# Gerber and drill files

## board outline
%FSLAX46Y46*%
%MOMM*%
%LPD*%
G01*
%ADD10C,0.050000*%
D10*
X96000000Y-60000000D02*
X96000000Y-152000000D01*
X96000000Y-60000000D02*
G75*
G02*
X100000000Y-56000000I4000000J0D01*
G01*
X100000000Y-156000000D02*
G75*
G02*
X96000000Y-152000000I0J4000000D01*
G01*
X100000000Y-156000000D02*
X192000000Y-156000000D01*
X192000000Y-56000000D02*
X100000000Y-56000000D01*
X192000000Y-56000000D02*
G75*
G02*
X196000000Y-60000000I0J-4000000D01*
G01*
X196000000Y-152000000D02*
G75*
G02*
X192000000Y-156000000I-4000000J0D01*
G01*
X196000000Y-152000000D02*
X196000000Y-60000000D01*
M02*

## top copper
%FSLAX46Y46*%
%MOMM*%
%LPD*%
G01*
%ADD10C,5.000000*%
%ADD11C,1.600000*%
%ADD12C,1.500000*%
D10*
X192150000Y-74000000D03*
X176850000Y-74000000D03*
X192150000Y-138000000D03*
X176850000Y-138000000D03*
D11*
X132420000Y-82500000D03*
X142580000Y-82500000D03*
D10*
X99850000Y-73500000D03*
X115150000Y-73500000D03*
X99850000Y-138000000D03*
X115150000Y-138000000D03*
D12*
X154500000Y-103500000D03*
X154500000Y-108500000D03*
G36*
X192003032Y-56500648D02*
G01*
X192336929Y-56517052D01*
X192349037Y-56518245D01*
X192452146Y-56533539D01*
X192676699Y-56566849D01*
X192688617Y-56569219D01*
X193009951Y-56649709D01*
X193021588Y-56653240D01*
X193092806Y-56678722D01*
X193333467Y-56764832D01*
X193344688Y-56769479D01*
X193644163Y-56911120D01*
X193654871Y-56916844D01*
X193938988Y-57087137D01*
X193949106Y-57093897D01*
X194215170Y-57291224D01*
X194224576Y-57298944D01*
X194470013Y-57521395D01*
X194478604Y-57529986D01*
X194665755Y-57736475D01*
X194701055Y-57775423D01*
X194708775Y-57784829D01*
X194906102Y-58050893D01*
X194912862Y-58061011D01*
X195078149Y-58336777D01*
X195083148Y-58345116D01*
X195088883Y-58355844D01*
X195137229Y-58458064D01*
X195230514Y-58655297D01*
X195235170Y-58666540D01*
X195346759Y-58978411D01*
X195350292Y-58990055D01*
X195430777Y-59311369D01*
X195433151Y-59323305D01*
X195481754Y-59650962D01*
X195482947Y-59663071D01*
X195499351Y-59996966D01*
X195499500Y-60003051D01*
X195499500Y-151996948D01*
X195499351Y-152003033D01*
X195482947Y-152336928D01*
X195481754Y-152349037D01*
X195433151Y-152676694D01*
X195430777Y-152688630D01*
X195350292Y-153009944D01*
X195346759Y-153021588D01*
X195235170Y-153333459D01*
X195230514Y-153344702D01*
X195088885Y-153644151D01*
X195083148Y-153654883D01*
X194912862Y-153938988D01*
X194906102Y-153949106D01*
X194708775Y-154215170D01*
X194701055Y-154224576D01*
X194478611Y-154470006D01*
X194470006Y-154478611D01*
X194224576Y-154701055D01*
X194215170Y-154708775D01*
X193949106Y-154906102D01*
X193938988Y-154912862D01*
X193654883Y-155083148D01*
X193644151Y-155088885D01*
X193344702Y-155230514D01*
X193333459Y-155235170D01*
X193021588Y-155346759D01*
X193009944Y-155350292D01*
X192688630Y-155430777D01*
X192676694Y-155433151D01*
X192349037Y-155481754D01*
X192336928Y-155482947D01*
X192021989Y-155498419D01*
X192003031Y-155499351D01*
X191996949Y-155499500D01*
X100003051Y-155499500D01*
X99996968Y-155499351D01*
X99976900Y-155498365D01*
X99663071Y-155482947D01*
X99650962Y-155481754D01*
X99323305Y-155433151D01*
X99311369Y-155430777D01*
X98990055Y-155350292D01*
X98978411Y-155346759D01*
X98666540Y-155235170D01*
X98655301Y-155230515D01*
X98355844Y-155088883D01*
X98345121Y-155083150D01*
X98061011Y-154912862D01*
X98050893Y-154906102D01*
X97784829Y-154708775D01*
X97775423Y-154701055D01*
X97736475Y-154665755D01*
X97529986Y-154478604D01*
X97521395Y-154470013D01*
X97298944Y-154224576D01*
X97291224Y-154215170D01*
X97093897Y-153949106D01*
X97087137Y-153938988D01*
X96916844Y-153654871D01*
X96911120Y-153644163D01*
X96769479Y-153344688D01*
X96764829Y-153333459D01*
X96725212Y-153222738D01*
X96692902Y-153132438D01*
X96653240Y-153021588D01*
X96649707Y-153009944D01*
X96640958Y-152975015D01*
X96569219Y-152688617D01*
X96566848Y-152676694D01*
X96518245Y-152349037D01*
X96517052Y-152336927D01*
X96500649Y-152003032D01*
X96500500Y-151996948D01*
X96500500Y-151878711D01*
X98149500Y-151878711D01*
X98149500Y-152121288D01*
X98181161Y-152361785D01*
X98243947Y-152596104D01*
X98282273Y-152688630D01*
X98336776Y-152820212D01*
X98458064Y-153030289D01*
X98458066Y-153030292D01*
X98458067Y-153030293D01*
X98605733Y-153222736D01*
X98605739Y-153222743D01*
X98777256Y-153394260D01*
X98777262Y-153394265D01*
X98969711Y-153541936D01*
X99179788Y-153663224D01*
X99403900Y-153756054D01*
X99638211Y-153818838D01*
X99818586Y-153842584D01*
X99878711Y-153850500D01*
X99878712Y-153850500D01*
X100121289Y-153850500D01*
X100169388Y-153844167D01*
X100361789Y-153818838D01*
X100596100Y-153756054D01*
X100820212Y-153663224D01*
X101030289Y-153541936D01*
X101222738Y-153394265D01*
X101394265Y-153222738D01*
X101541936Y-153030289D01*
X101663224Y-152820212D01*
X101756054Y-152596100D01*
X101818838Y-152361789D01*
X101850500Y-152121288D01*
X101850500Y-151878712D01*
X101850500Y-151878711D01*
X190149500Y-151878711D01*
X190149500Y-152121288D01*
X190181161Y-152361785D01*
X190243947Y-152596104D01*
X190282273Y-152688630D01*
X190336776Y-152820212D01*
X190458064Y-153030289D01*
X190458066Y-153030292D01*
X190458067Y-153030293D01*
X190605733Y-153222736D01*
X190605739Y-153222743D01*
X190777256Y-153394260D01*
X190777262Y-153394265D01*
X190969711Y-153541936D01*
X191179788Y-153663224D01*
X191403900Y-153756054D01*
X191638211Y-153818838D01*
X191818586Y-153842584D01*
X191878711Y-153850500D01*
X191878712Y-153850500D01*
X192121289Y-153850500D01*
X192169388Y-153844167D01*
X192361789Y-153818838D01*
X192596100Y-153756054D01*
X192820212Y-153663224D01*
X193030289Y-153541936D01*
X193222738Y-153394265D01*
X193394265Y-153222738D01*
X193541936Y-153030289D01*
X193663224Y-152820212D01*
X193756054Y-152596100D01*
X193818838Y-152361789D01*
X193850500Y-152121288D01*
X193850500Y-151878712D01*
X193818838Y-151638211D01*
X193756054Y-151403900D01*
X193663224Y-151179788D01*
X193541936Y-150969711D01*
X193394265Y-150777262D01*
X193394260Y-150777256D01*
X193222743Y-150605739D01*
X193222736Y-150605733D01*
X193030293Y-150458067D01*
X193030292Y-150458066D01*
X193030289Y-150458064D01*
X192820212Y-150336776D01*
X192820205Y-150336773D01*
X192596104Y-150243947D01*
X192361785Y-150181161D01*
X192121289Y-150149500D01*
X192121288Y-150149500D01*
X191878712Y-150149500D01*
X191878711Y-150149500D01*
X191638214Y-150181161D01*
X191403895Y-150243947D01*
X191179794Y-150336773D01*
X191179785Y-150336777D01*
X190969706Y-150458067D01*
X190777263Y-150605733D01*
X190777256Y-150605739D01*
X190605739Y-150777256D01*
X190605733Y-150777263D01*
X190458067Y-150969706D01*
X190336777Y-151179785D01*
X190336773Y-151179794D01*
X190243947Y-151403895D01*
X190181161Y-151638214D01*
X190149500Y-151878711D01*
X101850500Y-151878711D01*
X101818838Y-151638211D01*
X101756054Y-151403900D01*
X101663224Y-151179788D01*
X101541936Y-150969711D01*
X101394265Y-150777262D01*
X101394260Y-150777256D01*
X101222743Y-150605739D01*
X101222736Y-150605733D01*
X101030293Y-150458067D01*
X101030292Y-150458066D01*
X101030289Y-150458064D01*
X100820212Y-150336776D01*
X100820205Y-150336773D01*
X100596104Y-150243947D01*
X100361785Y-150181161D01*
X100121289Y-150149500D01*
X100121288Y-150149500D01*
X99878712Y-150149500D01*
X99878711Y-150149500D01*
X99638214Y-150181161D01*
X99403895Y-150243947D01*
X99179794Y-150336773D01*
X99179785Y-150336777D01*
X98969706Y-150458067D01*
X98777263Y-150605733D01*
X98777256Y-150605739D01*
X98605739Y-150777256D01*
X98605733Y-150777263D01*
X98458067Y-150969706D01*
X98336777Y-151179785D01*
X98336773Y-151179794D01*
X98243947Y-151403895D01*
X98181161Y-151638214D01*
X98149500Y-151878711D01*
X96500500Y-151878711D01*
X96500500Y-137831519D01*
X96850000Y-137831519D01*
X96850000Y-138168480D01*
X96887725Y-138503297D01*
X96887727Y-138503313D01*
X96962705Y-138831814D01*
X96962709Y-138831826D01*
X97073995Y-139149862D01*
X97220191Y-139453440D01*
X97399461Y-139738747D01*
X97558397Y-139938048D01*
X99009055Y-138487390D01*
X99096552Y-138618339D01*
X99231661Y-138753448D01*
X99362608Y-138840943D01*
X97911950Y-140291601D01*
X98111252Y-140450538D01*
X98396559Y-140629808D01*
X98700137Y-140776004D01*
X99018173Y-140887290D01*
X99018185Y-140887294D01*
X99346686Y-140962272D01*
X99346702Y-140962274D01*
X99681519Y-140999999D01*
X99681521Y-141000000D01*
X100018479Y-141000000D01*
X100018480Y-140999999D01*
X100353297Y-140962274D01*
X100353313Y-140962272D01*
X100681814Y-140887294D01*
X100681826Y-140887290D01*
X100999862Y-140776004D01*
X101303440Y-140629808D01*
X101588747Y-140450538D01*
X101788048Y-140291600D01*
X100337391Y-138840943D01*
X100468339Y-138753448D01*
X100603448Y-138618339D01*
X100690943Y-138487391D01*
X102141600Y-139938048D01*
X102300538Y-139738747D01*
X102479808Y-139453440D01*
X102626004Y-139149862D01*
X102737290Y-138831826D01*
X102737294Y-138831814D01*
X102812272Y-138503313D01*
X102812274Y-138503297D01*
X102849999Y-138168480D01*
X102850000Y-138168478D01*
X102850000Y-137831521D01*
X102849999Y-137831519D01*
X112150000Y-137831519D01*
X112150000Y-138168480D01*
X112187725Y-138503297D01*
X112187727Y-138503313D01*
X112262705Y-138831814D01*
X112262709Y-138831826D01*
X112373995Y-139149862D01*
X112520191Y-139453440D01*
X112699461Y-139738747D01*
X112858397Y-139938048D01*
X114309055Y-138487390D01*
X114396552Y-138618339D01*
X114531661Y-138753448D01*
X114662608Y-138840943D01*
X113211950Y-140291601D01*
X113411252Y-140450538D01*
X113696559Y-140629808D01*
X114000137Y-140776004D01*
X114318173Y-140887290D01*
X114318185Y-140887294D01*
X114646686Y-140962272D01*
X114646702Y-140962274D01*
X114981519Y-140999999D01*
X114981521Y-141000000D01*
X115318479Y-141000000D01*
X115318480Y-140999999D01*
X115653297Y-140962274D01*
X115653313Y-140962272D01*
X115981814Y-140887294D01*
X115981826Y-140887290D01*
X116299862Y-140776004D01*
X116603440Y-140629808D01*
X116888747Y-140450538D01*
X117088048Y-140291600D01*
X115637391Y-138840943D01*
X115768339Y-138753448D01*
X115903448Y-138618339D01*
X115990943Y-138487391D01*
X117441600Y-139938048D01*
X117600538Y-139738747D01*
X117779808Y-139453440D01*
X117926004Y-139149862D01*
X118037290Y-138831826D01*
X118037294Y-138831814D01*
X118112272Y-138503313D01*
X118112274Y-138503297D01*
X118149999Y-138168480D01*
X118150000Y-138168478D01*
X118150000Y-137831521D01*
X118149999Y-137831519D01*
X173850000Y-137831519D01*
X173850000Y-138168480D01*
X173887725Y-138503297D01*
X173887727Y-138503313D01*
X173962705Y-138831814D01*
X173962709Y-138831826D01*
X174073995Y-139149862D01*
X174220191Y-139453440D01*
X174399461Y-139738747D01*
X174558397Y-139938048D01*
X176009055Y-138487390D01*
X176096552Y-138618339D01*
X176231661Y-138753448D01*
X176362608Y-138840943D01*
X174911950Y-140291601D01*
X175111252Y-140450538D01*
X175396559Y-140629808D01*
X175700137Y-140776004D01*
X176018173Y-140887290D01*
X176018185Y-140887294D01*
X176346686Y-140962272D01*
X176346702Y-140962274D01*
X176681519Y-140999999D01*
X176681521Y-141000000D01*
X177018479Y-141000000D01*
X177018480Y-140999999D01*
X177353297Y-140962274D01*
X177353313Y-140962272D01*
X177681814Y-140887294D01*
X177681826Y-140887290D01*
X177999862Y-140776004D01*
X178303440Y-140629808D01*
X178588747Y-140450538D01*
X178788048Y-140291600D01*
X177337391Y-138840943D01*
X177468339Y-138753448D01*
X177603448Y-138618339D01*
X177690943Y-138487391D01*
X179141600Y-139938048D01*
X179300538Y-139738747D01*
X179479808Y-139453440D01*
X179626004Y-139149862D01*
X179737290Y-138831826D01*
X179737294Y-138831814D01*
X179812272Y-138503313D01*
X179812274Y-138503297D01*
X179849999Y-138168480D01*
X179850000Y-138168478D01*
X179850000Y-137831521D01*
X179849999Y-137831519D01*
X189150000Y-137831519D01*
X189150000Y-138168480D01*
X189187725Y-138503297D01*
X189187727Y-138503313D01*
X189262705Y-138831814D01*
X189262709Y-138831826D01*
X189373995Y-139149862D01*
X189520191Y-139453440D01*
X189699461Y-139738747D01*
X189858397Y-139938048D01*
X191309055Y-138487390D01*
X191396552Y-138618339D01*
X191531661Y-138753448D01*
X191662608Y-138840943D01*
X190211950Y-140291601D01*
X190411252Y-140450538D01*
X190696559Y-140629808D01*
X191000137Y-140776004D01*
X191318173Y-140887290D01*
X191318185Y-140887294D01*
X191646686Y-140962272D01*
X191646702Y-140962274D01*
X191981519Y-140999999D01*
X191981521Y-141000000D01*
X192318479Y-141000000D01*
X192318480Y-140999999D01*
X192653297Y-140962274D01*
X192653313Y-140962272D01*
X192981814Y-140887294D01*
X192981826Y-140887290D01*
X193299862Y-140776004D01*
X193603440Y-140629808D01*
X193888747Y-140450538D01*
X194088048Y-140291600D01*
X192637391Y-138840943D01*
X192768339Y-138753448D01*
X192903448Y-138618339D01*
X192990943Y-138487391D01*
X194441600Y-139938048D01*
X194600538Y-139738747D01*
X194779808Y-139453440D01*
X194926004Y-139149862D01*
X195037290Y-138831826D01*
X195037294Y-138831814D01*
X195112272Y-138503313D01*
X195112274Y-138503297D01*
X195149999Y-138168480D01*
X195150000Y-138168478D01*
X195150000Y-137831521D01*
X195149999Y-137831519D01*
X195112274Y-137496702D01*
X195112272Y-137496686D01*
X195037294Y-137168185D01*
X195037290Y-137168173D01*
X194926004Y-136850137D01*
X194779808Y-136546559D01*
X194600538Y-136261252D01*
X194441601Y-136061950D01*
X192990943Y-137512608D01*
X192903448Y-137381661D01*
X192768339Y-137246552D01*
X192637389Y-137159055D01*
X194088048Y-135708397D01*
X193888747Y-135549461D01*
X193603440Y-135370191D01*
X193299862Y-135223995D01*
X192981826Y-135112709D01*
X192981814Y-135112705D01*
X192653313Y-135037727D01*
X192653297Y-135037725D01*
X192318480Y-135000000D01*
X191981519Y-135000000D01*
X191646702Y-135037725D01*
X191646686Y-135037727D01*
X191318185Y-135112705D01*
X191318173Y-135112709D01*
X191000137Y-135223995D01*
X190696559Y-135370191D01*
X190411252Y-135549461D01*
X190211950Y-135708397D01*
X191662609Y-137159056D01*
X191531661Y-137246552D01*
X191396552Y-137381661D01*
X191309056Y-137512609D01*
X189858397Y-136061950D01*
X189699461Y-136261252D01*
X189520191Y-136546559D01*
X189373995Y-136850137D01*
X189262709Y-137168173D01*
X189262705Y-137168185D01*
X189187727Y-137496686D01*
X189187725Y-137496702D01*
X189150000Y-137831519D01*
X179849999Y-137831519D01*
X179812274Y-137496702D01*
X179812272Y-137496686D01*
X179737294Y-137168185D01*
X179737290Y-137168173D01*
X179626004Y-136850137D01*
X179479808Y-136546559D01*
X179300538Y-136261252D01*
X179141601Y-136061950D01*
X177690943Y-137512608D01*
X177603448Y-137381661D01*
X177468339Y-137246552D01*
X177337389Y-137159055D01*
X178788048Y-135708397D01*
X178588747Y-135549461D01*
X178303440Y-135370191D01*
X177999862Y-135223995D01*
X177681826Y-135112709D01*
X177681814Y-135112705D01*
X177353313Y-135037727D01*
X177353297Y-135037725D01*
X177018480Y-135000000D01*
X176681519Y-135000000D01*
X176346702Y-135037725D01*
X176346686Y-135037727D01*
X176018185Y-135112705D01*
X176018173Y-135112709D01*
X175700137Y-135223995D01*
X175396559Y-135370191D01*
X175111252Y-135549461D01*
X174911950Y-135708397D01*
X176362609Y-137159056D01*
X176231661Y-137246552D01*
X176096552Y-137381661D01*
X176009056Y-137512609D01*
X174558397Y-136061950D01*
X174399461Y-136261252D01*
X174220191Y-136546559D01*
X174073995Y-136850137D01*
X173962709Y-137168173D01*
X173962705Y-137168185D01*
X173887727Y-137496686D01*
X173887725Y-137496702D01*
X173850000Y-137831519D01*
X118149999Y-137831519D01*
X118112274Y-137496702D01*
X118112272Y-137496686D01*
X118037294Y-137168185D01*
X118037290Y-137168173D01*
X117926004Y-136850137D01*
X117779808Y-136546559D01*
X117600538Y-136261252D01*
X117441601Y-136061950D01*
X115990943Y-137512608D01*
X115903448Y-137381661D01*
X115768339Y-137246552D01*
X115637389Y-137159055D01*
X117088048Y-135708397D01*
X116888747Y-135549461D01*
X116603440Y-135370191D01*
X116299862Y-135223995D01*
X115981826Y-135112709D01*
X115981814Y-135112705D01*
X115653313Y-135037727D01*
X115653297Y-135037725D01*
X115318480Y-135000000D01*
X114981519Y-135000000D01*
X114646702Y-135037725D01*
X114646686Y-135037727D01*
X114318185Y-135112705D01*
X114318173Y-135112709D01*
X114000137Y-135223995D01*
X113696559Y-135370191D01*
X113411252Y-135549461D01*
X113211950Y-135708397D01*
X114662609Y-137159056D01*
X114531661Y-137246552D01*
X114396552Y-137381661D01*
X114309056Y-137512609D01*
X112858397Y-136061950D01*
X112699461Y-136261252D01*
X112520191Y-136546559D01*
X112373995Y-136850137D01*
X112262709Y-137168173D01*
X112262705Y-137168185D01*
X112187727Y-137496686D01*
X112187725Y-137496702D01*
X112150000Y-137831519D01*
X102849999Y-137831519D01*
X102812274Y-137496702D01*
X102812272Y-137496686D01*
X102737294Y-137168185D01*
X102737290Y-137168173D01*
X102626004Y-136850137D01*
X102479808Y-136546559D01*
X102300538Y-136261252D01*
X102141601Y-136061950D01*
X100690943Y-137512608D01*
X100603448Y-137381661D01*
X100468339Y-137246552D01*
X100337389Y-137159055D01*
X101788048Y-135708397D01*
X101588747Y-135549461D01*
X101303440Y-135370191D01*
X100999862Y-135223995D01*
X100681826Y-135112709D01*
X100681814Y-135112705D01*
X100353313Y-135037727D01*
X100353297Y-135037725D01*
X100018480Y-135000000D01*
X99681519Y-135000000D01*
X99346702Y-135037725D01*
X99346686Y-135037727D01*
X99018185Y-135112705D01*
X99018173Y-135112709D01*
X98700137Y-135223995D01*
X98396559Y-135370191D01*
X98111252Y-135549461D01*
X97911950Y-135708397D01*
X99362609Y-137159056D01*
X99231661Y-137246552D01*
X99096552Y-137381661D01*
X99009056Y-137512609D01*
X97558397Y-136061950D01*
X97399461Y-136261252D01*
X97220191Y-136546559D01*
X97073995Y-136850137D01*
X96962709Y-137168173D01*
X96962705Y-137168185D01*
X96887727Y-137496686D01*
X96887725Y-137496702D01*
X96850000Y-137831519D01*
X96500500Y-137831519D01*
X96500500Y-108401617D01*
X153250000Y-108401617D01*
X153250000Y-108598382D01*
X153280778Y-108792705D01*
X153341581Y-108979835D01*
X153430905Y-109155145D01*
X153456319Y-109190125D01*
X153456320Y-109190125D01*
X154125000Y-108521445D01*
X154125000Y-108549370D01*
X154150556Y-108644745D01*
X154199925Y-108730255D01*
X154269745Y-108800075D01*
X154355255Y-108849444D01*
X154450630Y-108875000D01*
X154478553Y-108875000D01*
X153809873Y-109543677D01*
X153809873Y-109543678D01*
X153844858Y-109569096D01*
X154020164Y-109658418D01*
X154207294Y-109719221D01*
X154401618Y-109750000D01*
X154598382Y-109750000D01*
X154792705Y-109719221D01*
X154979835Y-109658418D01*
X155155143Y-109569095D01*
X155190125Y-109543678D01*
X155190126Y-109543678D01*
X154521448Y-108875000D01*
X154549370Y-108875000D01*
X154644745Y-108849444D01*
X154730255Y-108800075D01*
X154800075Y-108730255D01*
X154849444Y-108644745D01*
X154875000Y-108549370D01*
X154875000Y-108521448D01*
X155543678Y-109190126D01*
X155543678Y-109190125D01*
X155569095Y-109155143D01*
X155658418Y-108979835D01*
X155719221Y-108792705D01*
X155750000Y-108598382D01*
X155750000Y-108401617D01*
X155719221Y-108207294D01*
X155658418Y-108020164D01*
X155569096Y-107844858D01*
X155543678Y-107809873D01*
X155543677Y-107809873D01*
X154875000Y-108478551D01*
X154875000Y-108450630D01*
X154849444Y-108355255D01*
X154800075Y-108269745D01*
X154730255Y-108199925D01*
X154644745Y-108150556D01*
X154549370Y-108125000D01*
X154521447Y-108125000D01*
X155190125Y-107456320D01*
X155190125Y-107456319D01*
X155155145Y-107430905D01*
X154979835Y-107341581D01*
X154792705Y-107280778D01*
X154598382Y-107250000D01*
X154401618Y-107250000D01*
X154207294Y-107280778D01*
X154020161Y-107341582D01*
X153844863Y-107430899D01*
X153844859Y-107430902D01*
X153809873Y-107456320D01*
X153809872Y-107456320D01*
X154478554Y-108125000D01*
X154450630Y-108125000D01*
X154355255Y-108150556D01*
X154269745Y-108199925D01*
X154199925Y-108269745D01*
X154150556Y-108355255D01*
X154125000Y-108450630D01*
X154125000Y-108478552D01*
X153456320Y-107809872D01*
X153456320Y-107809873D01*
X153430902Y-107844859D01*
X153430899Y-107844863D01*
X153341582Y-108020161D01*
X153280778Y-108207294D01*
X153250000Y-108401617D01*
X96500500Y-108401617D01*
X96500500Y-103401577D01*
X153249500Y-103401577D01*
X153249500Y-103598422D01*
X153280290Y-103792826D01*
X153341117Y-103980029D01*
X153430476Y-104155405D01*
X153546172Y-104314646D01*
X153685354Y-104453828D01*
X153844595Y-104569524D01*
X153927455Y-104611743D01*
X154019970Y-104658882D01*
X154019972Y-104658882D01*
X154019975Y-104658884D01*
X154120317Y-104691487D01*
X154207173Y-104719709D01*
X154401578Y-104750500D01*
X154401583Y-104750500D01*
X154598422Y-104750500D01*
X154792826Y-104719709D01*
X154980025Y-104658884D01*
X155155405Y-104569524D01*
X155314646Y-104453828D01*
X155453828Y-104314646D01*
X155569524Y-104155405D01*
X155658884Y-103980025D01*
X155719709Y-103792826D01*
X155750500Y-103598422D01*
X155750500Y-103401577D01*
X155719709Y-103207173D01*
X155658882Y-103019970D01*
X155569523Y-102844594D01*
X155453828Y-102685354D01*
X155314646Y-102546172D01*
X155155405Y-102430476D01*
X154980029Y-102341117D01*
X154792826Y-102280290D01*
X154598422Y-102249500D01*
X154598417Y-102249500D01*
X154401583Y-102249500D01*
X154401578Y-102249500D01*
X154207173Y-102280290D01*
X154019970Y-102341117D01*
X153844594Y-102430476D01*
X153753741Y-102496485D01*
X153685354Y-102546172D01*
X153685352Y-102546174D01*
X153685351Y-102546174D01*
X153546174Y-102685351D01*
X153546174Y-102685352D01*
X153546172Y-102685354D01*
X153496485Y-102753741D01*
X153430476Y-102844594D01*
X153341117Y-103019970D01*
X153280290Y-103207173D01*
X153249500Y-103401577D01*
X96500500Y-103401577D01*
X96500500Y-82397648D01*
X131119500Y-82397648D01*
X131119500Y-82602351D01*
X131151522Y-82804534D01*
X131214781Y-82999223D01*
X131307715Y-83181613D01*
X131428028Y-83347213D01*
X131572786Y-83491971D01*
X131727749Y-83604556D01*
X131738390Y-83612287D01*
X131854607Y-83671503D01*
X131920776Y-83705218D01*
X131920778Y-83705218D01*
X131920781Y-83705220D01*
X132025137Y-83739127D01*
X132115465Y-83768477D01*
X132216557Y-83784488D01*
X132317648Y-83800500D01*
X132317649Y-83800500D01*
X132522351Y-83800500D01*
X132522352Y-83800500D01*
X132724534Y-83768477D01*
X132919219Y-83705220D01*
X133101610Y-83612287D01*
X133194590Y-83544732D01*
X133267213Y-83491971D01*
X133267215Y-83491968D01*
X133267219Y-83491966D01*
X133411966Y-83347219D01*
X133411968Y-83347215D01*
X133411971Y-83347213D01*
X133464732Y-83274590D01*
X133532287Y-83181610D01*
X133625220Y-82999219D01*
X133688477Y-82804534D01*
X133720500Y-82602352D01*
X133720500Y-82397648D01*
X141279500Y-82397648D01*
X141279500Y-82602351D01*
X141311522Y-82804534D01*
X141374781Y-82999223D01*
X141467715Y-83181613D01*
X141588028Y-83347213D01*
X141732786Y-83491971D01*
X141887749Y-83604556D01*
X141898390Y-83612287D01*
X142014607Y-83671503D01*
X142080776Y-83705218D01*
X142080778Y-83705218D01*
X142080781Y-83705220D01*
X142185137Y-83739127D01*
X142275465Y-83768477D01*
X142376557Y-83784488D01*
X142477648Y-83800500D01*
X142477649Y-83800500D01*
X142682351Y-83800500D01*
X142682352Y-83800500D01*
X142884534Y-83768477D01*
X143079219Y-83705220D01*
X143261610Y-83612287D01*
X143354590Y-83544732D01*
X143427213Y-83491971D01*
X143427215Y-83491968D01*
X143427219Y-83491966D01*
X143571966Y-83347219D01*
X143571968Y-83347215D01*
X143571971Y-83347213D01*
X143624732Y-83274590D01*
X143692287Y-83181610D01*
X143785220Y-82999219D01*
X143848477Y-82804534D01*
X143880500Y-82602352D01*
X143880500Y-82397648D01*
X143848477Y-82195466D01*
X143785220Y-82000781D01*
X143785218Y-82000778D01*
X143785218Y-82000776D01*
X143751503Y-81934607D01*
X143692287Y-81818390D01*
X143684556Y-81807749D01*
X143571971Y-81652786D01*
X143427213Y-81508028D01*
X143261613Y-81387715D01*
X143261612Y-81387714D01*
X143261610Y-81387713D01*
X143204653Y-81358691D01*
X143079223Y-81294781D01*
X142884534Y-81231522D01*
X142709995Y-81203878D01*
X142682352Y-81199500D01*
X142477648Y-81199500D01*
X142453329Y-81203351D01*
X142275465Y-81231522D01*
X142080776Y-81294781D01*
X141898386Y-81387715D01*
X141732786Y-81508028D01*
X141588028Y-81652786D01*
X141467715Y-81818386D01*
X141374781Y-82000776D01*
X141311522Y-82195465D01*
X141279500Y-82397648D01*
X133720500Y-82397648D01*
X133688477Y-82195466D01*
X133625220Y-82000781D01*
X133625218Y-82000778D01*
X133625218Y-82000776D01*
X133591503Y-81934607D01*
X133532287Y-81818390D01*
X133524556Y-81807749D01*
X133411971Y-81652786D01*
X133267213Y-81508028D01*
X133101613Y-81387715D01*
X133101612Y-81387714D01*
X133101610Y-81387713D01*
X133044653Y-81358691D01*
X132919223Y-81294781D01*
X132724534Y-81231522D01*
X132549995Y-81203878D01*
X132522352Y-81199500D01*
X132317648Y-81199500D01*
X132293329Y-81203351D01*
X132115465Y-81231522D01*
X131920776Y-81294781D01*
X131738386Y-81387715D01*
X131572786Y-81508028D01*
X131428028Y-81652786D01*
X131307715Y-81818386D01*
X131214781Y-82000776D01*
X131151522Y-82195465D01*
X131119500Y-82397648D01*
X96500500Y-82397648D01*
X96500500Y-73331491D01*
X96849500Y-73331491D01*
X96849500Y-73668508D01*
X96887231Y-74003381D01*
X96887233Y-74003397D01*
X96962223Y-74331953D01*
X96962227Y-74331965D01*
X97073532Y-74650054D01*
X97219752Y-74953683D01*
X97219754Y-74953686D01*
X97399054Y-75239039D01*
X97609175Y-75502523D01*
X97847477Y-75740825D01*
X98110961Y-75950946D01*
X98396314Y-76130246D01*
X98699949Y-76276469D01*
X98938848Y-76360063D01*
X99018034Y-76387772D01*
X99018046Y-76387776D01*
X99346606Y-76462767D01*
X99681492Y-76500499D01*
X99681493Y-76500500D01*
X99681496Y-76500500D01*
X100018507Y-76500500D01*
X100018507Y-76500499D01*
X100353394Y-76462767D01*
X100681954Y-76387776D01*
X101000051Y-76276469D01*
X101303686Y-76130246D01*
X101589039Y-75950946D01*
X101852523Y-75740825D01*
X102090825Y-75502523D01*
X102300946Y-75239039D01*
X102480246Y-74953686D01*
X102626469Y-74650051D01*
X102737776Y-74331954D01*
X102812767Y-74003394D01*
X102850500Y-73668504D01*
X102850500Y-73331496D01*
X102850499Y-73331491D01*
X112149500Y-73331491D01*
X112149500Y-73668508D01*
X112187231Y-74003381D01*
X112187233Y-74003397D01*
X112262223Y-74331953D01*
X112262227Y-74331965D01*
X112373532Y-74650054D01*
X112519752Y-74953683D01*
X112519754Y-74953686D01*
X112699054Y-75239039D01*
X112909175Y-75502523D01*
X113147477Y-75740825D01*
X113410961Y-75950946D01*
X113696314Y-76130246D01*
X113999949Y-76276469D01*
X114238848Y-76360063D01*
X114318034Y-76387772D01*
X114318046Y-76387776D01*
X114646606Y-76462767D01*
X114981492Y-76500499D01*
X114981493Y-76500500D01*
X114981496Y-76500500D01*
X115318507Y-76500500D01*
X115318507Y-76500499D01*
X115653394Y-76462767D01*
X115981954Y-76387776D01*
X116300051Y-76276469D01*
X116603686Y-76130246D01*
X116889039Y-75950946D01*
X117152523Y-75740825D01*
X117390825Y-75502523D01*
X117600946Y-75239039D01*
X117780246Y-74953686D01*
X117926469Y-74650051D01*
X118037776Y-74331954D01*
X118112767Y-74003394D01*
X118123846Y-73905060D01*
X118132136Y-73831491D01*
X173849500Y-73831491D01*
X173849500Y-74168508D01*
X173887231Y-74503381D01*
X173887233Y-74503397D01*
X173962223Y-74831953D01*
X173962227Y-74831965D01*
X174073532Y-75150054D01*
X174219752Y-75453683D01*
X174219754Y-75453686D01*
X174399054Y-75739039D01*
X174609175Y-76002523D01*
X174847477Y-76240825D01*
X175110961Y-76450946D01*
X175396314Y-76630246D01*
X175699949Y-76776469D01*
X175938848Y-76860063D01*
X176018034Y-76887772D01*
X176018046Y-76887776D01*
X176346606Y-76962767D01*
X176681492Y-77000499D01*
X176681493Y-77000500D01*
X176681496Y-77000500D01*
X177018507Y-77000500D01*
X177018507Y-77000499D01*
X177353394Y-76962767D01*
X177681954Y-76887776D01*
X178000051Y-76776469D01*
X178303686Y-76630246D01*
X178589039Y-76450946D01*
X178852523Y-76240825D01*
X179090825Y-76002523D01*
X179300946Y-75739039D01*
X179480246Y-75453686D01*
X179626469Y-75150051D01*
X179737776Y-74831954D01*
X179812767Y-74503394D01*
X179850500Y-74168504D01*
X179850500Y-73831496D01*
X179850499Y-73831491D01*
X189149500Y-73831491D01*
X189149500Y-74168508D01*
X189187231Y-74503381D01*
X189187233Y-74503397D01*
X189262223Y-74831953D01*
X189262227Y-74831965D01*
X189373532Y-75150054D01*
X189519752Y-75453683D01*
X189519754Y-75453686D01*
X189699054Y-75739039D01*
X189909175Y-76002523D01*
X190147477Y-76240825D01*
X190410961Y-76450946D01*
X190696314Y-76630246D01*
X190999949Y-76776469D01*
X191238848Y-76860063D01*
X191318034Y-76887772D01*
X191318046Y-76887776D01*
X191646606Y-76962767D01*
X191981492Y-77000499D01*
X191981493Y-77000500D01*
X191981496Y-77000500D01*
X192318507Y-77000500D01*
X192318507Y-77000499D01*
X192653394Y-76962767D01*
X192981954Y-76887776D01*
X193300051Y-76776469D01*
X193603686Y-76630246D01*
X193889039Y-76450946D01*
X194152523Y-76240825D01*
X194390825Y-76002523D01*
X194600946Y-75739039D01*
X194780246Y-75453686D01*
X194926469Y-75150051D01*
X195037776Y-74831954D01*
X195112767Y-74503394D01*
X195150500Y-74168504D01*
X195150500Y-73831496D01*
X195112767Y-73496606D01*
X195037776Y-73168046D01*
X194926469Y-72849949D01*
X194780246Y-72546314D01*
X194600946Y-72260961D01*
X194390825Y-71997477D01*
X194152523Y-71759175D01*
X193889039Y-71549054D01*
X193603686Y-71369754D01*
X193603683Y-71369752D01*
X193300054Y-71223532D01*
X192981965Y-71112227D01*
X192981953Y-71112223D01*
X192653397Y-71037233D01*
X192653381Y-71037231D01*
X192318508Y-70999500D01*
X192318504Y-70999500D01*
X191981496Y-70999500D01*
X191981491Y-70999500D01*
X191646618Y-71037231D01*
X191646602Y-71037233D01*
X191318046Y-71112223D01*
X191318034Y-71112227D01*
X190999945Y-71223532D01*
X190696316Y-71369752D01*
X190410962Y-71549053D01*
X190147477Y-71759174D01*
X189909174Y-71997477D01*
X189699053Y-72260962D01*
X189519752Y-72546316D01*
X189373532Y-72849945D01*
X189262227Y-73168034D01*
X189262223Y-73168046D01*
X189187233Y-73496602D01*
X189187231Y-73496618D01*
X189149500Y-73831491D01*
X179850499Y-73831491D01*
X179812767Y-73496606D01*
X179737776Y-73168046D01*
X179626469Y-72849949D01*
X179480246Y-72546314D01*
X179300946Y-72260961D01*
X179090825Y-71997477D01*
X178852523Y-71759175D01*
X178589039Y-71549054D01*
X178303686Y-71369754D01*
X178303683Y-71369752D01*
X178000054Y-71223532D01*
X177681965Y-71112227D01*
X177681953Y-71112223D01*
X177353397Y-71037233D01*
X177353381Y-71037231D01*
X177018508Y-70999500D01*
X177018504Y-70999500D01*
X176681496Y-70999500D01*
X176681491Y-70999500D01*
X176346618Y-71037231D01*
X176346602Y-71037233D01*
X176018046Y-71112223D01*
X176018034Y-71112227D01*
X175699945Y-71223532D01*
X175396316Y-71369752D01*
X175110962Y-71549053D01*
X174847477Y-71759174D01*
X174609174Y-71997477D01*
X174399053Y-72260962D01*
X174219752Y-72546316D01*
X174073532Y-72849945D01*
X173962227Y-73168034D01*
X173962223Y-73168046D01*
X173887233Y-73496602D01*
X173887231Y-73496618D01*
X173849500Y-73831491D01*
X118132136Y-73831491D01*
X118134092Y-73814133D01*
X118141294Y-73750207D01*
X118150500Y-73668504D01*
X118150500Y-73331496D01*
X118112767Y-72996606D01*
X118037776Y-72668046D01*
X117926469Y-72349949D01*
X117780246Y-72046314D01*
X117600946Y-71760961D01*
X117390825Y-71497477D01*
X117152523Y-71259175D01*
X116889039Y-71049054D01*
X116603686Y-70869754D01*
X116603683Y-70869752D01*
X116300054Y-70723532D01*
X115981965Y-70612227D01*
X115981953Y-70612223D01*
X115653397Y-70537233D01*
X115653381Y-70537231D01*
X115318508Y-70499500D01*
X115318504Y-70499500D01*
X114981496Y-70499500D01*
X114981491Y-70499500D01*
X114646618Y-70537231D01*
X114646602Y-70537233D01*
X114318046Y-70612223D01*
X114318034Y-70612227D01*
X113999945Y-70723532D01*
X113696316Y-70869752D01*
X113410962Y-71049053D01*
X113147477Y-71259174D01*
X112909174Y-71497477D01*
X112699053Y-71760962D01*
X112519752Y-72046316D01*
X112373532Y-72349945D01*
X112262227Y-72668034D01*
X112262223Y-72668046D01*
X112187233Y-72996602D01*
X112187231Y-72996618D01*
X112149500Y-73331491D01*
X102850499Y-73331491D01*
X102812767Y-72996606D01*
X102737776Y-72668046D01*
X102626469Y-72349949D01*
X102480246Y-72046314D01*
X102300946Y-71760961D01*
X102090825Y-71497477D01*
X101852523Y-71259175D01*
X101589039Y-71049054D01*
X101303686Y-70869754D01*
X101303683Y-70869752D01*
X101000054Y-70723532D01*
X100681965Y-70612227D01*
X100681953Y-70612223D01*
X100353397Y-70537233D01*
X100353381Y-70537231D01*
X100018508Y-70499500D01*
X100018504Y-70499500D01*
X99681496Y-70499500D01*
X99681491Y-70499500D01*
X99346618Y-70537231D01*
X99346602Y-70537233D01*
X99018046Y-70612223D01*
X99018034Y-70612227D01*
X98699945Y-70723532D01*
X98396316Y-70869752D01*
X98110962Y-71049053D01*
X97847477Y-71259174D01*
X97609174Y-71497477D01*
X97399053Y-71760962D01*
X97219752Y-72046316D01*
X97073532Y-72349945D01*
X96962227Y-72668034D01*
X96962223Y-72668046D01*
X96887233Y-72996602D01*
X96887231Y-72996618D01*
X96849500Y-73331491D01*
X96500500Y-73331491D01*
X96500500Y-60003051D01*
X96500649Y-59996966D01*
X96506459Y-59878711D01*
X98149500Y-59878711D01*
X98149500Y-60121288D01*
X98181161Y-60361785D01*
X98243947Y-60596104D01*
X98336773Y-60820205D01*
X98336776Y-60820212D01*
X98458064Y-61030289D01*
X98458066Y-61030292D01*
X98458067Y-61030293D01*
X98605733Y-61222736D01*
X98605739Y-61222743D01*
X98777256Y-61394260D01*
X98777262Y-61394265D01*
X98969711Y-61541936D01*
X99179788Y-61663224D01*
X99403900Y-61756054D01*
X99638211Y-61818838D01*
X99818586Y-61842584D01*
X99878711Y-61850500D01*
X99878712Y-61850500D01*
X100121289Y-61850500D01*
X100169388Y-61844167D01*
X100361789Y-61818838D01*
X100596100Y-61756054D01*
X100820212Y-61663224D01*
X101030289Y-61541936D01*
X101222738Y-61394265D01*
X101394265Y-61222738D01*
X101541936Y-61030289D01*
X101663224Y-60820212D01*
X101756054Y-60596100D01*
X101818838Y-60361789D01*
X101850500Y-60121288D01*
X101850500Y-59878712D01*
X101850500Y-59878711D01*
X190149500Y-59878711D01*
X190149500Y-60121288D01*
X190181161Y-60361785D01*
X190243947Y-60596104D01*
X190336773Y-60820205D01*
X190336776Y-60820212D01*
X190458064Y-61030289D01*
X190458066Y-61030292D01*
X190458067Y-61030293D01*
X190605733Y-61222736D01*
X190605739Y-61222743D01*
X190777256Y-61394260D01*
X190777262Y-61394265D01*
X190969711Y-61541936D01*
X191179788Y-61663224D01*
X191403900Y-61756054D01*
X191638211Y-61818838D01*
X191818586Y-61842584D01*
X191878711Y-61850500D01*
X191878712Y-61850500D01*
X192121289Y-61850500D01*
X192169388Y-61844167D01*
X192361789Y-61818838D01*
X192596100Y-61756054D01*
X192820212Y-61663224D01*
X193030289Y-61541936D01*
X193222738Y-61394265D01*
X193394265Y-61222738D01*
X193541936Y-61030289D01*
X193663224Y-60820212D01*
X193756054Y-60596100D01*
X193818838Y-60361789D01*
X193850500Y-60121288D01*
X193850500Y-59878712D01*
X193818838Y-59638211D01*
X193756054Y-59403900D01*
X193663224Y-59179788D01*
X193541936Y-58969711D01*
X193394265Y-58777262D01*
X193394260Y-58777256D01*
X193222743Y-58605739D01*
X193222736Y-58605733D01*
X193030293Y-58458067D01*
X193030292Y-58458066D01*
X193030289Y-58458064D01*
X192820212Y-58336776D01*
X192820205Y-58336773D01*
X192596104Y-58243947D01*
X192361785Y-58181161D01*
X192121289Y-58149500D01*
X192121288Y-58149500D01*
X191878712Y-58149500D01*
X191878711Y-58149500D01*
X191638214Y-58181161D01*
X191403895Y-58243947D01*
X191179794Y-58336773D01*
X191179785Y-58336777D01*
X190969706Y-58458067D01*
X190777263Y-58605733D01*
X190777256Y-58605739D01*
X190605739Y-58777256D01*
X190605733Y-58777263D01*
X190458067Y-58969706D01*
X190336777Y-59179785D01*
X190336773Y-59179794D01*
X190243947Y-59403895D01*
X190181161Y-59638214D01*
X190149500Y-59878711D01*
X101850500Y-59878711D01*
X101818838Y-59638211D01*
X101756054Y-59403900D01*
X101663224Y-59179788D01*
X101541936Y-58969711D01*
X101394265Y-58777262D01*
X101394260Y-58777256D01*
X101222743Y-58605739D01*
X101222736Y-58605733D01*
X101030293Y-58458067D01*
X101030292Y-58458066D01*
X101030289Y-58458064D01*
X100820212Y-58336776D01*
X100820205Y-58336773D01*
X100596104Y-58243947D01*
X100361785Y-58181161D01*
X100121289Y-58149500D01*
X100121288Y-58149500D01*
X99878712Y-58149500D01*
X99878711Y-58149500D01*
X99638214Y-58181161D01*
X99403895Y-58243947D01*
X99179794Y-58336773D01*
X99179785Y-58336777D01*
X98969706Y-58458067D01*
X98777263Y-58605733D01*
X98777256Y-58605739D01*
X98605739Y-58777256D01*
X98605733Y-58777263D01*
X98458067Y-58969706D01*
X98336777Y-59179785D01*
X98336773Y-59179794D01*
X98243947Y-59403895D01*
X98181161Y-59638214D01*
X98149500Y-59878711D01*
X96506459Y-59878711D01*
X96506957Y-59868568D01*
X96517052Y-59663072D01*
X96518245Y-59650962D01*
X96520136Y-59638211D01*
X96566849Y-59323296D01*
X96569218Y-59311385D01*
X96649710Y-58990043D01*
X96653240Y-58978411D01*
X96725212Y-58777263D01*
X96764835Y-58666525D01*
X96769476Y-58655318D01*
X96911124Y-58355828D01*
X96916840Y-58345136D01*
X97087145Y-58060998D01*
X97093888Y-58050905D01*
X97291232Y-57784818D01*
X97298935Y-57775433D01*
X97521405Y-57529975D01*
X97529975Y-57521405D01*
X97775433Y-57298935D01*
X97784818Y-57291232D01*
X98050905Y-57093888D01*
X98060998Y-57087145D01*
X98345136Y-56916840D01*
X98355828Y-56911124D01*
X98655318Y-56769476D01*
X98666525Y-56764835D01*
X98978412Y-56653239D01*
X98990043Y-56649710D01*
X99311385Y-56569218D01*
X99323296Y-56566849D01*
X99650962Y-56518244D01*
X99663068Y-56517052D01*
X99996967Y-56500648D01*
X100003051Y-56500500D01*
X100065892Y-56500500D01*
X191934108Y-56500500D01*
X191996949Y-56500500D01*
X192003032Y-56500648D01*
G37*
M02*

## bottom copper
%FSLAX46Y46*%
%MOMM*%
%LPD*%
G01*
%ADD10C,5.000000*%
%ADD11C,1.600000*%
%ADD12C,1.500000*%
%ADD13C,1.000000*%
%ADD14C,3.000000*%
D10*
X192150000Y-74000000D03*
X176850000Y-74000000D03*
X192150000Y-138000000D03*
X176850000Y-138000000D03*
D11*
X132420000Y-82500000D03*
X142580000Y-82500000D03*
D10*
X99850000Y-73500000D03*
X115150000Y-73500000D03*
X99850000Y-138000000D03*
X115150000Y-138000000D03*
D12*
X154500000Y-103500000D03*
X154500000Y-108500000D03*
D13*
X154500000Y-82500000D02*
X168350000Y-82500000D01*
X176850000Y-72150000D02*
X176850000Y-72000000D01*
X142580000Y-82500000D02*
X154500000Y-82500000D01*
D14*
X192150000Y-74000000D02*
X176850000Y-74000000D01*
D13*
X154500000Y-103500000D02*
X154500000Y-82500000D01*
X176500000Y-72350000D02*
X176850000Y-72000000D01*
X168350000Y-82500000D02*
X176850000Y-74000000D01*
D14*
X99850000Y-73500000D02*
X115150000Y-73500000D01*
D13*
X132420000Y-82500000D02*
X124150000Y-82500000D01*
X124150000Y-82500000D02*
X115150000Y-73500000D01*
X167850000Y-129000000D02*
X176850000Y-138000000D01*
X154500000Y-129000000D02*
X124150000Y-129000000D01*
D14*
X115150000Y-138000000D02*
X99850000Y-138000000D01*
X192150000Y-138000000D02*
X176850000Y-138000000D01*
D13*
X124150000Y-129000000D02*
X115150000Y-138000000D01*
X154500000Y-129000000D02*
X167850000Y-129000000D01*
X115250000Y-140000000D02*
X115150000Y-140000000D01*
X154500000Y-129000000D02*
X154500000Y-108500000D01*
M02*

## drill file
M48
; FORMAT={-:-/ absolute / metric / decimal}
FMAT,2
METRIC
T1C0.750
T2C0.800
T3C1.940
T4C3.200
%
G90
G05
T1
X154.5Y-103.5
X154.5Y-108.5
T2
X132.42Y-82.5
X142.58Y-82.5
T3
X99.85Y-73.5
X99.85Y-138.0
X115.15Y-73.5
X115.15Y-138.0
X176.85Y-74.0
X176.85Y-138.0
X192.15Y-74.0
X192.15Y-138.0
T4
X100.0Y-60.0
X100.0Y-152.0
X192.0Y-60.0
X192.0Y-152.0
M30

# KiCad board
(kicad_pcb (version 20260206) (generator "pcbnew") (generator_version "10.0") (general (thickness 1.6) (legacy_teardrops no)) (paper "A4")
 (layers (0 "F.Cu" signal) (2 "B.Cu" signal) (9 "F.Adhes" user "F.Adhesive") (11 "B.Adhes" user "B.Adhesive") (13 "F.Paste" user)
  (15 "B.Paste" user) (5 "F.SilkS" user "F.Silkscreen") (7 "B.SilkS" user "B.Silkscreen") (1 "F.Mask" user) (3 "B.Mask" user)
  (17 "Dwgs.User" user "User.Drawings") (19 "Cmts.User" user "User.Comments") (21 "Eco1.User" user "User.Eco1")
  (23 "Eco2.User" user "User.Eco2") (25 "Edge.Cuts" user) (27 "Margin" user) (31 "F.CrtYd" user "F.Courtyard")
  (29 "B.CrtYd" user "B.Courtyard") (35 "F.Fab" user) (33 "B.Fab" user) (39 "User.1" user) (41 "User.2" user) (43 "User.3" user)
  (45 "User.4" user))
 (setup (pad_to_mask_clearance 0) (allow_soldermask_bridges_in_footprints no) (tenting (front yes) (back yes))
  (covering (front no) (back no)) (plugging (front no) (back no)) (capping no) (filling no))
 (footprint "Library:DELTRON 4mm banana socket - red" (layer "F.Cu") (at 184.5 74 180)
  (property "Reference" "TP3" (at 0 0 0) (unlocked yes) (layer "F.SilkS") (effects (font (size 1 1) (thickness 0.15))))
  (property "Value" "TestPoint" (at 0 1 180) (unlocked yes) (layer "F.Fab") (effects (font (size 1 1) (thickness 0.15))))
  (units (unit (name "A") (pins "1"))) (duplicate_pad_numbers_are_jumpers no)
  (pad "1" thru_hole circle (at -7.65 0 180) (size 5 5) (drill 1.94) (layers "*.Cu" "*.Mask") (remove_unused_layers no)
   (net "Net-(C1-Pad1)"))
  (pad "1" thru_hole circle (at 7.65 0 180) (size 5 5) (drill 1.94) (layers "*.Cu" "*.Mask") (remove_unused_layers no) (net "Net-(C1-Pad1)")))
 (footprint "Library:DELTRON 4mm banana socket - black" (layer "F.Cu") (at 184.5 138 180)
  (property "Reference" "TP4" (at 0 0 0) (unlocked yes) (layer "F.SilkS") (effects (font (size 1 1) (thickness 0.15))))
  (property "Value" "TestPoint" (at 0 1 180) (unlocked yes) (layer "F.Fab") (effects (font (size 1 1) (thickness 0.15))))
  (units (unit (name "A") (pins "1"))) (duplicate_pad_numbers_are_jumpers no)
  (pad "1" thru_hole circle (at -7.65 0 180) (size 5 5) (drill 1.94) (layers "*.Cu" "*.Mask") (remove_unused_layers no) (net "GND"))
  (pad "1" thru_hole circle (at 7.65 0 180) (size 5 5) (drill 1.94) (layers "*.Cu" "*.Mask") (remove_unused_layers no) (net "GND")))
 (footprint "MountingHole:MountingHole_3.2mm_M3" (layer "F.Cu") (at 192 152)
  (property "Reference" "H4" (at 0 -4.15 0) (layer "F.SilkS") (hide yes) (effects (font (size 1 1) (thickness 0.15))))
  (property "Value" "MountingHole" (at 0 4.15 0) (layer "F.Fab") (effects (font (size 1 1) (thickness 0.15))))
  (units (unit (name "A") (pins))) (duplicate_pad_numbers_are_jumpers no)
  (pad "" np_thru_hole circle (at 0 0) (size 3.2 3.2) (drill 3.2) (layers "*.Cu" "*.Mask")))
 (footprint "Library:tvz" (layer "F.Cu") (at 175.5 150)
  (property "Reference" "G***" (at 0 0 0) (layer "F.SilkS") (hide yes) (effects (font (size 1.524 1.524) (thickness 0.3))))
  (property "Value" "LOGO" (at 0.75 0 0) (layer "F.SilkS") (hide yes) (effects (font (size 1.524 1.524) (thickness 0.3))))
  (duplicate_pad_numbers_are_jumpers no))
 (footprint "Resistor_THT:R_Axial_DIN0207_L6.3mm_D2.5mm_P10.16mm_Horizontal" (layer "F.Cu") (at 132.42 82.5)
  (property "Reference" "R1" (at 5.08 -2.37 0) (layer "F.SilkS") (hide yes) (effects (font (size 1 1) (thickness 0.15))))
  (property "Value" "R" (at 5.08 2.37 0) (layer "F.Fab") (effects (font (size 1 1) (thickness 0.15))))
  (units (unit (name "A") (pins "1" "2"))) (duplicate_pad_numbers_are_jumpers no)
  (pad "1" thru_hole circle (at 0 0) (size 1.6 1.6) (drill 0.8) (layers "*.Cu" "*.Mask") (remove_unused_layers no) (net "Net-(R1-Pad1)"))
  (pad "2" thru_hole circle (at 10.16 0) (size 1.6 1.6) (drill 0.8) (layers "*.Cu" "*.Mask") (remove_unused_layers no) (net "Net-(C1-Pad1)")))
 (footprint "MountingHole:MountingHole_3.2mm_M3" (layer "F.Cu") (at 100 152)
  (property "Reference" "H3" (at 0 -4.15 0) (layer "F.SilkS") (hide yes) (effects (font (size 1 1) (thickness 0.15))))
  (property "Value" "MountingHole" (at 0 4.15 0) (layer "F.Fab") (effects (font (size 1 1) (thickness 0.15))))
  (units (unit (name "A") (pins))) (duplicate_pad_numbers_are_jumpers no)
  (pad "" np_thru_hole circle (at 0 0) (size 3.2 3.2) (drill 3.2) (layers "*.Cu" "*.Mask")))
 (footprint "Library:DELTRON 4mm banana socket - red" (layer "F.Cu") (at 107.5 73.5)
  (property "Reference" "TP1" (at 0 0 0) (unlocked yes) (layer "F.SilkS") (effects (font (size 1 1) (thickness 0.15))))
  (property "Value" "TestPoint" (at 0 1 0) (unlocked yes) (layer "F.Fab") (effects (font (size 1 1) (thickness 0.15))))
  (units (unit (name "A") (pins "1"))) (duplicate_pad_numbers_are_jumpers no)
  (pad "1" thru_hole circle (at -7.65 0) (size 5 5) (drill 1.94) (layers "*.Cu" "*.Mask") (remove_unused_layers no) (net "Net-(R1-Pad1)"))
  (pad "1" thru_hole circle (at 7.65 0) (size 5 5) (drill 1.94) (layers "*.Cu" "*.Mask") (remove_unused_layers no) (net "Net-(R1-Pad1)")))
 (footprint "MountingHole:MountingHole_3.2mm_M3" (layer "F.Cu") (at 100 60)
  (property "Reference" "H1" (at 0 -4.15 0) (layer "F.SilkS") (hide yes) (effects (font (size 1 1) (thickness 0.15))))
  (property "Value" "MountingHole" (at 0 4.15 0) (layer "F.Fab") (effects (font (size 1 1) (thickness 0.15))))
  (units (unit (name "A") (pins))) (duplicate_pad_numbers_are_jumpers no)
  (pad "" np_thru_hole circle (at 0 0) (size 3.2 3.2) (drill 3.2) (layers "*.Cu" "*.Mask")))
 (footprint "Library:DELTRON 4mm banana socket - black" (layer "F.Cu") (at 107.5 138)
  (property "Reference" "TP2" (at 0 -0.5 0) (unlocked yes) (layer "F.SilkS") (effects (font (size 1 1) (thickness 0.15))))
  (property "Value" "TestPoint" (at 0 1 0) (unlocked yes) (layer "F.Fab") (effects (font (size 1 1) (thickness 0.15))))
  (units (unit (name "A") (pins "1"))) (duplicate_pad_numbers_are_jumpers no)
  (pad "1" thru_hole circle (at -7.65 0) (size 5 5) (drill 1.94) (layers "*.Cu" "*.Mask") (remove_unused_layers no) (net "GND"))
  (pad "1" thru_hole circle (at 7.65 0) (size 5 5) (drill 1.94) (layers "*.Cu" "*.Mask") (remove_unused_layers no) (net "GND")))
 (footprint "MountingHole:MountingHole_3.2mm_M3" (layer "F.Cu") (at 192 60)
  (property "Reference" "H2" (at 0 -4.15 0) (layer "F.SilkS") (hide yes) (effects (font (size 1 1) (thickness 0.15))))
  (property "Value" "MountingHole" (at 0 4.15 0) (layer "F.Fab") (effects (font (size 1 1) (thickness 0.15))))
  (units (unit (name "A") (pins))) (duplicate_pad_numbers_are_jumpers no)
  (pad "" np_thru_hole circle (at 0 0) (size 3.2 3.2) (drill 3.2) (layers "*.Cu" "*.Mask")))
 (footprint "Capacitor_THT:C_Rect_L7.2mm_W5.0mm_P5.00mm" (layer "F.Cu") (at 154.5 103.5 -90)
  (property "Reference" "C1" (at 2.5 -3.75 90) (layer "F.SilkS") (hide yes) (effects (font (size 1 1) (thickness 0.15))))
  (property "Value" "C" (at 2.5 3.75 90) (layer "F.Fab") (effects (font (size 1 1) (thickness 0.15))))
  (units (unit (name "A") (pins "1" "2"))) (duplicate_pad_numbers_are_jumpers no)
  (pad "1" thru_hole circle (at 0 0 270) (size 1.5 1.5) (drill 0.75) (layers "*.Cu" "*.Mask") (remove_unused_layers no)
   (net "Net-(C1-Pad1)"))
  (pad "2" thru_hole circle (at 5 0 270) (size 1.5 1.5) (drill 0.75) (layers "*.Cu" "*.Mask") (remove_unused_layers no) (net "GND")))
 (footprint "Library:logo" (layer "B.Cu") (at 180.5 149 180)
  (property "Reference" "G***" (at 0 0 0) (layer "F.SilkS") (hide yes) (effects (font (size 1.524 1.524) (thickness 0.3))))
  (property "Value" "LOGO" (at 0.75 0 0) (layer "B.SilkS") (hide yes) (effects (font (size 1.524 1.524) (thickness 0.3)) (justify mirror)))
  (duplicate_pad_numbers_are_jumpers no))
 (gr_line (start 96 60) (end 96 152) (stroke (width 0.05) (type default)) (layer "Edge.Cuts"))
 (gr_arc (start 96 60) (mid 97.171573 57.171573) (end 100 56) (stroke (width 0.05) (type default)) (layer "Edge.Cuts"))
 (gr_arc (start 100 156) (mid 97.171573 154.828427) (end 96 152) (stroke (width 0.05) (type default)) (layer "Edge.Cuts"))
 (gr_line (start 100 156) (end 192 156) (stroke (width 0.05) (type default)) (layer "Edge.Cuts"))
 (gr_line (start 192 56) (end 100 56) (stroke (width 0.05) (type default)) (layer "Edge.Cuts"))
 (gr_arc (start 192 56) (mid 194.828427 57.171573) (end 196 60) (stroke (width 0.05) (type default)) (layer "Edge.Cuts"))
 (gr_arc (start 196 152) (mid 194.828427 154.828427) (end 192 156) (stroke (width 0.05) (type default)) (layer "Edge.Cuts"))
 (gr_line (start 196 152) (end 196 60) (stroke (width 0.05) (type default)) (layer "Edge.Cuts"))
 (segment (start 154.5 82.5) (end 168.35 82.5) (width 1) (layer "B.Cu") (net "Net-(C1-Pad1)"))
 (segment (start 176.85 72.15) (end 176.85 72) (width 1) (layer "B.Cu") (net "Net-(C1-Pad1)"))
 (segment (start 142.58 82.5) (end 154.5 82.5) (width 1) (layer "B.Cu") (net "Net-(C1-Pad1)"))
 (segment (start 192.15 74) (end 176.85 74) (width 3) (layer "B.Cu") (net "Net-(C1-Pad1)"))
 (segment (start 154.5 103.5) (end 154.5 82.5) (width 1) (layer "B.Cu") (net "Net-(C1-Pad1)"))
 (segment (start 176.5 72.35) (end 176.85 72) (width 1) (layer "B.Cu") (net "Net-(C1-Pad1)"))
 (segment (start 168.35 82.5) (end 176.85 74) (width 1) (layer "B.Cu") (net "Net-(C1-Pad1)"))
 (segment (start 99.85 73.5) (end 115.15 73.5) (width 3) (layer "B.Cu") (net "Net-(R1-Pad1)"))
 (segment (start 132.42 82.5) (end 124.15 82.5) (width 1) (layer "B.Cu") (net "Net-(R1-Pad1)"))
 (segment (start 124.15 82.5) (end 115.15 73.5) (width 1) (layer "B.Cu") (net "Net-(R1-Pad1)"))
 (segment (start 167.85 129) (end 176.85 138) (width 1) (layer "B.Cu") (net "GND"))
 (segment (start 154.5 129) (end 124.15 129) (width 1) (layer "B.Cu") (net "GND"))
 (segment (start 115.15 138) (end 99.85 138) (width 3) (layer "B.Cu") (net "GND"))
 (segment (start 192.15 138) (end 176.85 138) (width 3) (layer "B.Cu") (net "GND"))
 (segment (start 124.15 129) (end 115.15 138) (width 1) (layer "B.Cu") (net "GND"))
 (segment (start 154.5 129) (end 167.85 129) (width 1) (layer "B.Cu") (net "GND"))
 (segment (start 115.25 140) (end 115.15 140) (width 1) (layer "B.Cu") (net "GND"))
 (segment (start 154.5 129) (end 154.5 108.5) (width 1) (layer "B.Cu") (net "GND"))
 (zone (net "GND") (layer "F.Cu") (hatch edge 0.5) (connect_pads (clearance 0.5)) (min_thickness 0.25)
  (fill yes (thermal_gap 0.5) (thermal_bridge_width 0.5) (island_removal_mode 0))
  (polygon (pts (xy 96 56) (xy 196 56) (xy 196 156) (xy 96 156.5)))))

